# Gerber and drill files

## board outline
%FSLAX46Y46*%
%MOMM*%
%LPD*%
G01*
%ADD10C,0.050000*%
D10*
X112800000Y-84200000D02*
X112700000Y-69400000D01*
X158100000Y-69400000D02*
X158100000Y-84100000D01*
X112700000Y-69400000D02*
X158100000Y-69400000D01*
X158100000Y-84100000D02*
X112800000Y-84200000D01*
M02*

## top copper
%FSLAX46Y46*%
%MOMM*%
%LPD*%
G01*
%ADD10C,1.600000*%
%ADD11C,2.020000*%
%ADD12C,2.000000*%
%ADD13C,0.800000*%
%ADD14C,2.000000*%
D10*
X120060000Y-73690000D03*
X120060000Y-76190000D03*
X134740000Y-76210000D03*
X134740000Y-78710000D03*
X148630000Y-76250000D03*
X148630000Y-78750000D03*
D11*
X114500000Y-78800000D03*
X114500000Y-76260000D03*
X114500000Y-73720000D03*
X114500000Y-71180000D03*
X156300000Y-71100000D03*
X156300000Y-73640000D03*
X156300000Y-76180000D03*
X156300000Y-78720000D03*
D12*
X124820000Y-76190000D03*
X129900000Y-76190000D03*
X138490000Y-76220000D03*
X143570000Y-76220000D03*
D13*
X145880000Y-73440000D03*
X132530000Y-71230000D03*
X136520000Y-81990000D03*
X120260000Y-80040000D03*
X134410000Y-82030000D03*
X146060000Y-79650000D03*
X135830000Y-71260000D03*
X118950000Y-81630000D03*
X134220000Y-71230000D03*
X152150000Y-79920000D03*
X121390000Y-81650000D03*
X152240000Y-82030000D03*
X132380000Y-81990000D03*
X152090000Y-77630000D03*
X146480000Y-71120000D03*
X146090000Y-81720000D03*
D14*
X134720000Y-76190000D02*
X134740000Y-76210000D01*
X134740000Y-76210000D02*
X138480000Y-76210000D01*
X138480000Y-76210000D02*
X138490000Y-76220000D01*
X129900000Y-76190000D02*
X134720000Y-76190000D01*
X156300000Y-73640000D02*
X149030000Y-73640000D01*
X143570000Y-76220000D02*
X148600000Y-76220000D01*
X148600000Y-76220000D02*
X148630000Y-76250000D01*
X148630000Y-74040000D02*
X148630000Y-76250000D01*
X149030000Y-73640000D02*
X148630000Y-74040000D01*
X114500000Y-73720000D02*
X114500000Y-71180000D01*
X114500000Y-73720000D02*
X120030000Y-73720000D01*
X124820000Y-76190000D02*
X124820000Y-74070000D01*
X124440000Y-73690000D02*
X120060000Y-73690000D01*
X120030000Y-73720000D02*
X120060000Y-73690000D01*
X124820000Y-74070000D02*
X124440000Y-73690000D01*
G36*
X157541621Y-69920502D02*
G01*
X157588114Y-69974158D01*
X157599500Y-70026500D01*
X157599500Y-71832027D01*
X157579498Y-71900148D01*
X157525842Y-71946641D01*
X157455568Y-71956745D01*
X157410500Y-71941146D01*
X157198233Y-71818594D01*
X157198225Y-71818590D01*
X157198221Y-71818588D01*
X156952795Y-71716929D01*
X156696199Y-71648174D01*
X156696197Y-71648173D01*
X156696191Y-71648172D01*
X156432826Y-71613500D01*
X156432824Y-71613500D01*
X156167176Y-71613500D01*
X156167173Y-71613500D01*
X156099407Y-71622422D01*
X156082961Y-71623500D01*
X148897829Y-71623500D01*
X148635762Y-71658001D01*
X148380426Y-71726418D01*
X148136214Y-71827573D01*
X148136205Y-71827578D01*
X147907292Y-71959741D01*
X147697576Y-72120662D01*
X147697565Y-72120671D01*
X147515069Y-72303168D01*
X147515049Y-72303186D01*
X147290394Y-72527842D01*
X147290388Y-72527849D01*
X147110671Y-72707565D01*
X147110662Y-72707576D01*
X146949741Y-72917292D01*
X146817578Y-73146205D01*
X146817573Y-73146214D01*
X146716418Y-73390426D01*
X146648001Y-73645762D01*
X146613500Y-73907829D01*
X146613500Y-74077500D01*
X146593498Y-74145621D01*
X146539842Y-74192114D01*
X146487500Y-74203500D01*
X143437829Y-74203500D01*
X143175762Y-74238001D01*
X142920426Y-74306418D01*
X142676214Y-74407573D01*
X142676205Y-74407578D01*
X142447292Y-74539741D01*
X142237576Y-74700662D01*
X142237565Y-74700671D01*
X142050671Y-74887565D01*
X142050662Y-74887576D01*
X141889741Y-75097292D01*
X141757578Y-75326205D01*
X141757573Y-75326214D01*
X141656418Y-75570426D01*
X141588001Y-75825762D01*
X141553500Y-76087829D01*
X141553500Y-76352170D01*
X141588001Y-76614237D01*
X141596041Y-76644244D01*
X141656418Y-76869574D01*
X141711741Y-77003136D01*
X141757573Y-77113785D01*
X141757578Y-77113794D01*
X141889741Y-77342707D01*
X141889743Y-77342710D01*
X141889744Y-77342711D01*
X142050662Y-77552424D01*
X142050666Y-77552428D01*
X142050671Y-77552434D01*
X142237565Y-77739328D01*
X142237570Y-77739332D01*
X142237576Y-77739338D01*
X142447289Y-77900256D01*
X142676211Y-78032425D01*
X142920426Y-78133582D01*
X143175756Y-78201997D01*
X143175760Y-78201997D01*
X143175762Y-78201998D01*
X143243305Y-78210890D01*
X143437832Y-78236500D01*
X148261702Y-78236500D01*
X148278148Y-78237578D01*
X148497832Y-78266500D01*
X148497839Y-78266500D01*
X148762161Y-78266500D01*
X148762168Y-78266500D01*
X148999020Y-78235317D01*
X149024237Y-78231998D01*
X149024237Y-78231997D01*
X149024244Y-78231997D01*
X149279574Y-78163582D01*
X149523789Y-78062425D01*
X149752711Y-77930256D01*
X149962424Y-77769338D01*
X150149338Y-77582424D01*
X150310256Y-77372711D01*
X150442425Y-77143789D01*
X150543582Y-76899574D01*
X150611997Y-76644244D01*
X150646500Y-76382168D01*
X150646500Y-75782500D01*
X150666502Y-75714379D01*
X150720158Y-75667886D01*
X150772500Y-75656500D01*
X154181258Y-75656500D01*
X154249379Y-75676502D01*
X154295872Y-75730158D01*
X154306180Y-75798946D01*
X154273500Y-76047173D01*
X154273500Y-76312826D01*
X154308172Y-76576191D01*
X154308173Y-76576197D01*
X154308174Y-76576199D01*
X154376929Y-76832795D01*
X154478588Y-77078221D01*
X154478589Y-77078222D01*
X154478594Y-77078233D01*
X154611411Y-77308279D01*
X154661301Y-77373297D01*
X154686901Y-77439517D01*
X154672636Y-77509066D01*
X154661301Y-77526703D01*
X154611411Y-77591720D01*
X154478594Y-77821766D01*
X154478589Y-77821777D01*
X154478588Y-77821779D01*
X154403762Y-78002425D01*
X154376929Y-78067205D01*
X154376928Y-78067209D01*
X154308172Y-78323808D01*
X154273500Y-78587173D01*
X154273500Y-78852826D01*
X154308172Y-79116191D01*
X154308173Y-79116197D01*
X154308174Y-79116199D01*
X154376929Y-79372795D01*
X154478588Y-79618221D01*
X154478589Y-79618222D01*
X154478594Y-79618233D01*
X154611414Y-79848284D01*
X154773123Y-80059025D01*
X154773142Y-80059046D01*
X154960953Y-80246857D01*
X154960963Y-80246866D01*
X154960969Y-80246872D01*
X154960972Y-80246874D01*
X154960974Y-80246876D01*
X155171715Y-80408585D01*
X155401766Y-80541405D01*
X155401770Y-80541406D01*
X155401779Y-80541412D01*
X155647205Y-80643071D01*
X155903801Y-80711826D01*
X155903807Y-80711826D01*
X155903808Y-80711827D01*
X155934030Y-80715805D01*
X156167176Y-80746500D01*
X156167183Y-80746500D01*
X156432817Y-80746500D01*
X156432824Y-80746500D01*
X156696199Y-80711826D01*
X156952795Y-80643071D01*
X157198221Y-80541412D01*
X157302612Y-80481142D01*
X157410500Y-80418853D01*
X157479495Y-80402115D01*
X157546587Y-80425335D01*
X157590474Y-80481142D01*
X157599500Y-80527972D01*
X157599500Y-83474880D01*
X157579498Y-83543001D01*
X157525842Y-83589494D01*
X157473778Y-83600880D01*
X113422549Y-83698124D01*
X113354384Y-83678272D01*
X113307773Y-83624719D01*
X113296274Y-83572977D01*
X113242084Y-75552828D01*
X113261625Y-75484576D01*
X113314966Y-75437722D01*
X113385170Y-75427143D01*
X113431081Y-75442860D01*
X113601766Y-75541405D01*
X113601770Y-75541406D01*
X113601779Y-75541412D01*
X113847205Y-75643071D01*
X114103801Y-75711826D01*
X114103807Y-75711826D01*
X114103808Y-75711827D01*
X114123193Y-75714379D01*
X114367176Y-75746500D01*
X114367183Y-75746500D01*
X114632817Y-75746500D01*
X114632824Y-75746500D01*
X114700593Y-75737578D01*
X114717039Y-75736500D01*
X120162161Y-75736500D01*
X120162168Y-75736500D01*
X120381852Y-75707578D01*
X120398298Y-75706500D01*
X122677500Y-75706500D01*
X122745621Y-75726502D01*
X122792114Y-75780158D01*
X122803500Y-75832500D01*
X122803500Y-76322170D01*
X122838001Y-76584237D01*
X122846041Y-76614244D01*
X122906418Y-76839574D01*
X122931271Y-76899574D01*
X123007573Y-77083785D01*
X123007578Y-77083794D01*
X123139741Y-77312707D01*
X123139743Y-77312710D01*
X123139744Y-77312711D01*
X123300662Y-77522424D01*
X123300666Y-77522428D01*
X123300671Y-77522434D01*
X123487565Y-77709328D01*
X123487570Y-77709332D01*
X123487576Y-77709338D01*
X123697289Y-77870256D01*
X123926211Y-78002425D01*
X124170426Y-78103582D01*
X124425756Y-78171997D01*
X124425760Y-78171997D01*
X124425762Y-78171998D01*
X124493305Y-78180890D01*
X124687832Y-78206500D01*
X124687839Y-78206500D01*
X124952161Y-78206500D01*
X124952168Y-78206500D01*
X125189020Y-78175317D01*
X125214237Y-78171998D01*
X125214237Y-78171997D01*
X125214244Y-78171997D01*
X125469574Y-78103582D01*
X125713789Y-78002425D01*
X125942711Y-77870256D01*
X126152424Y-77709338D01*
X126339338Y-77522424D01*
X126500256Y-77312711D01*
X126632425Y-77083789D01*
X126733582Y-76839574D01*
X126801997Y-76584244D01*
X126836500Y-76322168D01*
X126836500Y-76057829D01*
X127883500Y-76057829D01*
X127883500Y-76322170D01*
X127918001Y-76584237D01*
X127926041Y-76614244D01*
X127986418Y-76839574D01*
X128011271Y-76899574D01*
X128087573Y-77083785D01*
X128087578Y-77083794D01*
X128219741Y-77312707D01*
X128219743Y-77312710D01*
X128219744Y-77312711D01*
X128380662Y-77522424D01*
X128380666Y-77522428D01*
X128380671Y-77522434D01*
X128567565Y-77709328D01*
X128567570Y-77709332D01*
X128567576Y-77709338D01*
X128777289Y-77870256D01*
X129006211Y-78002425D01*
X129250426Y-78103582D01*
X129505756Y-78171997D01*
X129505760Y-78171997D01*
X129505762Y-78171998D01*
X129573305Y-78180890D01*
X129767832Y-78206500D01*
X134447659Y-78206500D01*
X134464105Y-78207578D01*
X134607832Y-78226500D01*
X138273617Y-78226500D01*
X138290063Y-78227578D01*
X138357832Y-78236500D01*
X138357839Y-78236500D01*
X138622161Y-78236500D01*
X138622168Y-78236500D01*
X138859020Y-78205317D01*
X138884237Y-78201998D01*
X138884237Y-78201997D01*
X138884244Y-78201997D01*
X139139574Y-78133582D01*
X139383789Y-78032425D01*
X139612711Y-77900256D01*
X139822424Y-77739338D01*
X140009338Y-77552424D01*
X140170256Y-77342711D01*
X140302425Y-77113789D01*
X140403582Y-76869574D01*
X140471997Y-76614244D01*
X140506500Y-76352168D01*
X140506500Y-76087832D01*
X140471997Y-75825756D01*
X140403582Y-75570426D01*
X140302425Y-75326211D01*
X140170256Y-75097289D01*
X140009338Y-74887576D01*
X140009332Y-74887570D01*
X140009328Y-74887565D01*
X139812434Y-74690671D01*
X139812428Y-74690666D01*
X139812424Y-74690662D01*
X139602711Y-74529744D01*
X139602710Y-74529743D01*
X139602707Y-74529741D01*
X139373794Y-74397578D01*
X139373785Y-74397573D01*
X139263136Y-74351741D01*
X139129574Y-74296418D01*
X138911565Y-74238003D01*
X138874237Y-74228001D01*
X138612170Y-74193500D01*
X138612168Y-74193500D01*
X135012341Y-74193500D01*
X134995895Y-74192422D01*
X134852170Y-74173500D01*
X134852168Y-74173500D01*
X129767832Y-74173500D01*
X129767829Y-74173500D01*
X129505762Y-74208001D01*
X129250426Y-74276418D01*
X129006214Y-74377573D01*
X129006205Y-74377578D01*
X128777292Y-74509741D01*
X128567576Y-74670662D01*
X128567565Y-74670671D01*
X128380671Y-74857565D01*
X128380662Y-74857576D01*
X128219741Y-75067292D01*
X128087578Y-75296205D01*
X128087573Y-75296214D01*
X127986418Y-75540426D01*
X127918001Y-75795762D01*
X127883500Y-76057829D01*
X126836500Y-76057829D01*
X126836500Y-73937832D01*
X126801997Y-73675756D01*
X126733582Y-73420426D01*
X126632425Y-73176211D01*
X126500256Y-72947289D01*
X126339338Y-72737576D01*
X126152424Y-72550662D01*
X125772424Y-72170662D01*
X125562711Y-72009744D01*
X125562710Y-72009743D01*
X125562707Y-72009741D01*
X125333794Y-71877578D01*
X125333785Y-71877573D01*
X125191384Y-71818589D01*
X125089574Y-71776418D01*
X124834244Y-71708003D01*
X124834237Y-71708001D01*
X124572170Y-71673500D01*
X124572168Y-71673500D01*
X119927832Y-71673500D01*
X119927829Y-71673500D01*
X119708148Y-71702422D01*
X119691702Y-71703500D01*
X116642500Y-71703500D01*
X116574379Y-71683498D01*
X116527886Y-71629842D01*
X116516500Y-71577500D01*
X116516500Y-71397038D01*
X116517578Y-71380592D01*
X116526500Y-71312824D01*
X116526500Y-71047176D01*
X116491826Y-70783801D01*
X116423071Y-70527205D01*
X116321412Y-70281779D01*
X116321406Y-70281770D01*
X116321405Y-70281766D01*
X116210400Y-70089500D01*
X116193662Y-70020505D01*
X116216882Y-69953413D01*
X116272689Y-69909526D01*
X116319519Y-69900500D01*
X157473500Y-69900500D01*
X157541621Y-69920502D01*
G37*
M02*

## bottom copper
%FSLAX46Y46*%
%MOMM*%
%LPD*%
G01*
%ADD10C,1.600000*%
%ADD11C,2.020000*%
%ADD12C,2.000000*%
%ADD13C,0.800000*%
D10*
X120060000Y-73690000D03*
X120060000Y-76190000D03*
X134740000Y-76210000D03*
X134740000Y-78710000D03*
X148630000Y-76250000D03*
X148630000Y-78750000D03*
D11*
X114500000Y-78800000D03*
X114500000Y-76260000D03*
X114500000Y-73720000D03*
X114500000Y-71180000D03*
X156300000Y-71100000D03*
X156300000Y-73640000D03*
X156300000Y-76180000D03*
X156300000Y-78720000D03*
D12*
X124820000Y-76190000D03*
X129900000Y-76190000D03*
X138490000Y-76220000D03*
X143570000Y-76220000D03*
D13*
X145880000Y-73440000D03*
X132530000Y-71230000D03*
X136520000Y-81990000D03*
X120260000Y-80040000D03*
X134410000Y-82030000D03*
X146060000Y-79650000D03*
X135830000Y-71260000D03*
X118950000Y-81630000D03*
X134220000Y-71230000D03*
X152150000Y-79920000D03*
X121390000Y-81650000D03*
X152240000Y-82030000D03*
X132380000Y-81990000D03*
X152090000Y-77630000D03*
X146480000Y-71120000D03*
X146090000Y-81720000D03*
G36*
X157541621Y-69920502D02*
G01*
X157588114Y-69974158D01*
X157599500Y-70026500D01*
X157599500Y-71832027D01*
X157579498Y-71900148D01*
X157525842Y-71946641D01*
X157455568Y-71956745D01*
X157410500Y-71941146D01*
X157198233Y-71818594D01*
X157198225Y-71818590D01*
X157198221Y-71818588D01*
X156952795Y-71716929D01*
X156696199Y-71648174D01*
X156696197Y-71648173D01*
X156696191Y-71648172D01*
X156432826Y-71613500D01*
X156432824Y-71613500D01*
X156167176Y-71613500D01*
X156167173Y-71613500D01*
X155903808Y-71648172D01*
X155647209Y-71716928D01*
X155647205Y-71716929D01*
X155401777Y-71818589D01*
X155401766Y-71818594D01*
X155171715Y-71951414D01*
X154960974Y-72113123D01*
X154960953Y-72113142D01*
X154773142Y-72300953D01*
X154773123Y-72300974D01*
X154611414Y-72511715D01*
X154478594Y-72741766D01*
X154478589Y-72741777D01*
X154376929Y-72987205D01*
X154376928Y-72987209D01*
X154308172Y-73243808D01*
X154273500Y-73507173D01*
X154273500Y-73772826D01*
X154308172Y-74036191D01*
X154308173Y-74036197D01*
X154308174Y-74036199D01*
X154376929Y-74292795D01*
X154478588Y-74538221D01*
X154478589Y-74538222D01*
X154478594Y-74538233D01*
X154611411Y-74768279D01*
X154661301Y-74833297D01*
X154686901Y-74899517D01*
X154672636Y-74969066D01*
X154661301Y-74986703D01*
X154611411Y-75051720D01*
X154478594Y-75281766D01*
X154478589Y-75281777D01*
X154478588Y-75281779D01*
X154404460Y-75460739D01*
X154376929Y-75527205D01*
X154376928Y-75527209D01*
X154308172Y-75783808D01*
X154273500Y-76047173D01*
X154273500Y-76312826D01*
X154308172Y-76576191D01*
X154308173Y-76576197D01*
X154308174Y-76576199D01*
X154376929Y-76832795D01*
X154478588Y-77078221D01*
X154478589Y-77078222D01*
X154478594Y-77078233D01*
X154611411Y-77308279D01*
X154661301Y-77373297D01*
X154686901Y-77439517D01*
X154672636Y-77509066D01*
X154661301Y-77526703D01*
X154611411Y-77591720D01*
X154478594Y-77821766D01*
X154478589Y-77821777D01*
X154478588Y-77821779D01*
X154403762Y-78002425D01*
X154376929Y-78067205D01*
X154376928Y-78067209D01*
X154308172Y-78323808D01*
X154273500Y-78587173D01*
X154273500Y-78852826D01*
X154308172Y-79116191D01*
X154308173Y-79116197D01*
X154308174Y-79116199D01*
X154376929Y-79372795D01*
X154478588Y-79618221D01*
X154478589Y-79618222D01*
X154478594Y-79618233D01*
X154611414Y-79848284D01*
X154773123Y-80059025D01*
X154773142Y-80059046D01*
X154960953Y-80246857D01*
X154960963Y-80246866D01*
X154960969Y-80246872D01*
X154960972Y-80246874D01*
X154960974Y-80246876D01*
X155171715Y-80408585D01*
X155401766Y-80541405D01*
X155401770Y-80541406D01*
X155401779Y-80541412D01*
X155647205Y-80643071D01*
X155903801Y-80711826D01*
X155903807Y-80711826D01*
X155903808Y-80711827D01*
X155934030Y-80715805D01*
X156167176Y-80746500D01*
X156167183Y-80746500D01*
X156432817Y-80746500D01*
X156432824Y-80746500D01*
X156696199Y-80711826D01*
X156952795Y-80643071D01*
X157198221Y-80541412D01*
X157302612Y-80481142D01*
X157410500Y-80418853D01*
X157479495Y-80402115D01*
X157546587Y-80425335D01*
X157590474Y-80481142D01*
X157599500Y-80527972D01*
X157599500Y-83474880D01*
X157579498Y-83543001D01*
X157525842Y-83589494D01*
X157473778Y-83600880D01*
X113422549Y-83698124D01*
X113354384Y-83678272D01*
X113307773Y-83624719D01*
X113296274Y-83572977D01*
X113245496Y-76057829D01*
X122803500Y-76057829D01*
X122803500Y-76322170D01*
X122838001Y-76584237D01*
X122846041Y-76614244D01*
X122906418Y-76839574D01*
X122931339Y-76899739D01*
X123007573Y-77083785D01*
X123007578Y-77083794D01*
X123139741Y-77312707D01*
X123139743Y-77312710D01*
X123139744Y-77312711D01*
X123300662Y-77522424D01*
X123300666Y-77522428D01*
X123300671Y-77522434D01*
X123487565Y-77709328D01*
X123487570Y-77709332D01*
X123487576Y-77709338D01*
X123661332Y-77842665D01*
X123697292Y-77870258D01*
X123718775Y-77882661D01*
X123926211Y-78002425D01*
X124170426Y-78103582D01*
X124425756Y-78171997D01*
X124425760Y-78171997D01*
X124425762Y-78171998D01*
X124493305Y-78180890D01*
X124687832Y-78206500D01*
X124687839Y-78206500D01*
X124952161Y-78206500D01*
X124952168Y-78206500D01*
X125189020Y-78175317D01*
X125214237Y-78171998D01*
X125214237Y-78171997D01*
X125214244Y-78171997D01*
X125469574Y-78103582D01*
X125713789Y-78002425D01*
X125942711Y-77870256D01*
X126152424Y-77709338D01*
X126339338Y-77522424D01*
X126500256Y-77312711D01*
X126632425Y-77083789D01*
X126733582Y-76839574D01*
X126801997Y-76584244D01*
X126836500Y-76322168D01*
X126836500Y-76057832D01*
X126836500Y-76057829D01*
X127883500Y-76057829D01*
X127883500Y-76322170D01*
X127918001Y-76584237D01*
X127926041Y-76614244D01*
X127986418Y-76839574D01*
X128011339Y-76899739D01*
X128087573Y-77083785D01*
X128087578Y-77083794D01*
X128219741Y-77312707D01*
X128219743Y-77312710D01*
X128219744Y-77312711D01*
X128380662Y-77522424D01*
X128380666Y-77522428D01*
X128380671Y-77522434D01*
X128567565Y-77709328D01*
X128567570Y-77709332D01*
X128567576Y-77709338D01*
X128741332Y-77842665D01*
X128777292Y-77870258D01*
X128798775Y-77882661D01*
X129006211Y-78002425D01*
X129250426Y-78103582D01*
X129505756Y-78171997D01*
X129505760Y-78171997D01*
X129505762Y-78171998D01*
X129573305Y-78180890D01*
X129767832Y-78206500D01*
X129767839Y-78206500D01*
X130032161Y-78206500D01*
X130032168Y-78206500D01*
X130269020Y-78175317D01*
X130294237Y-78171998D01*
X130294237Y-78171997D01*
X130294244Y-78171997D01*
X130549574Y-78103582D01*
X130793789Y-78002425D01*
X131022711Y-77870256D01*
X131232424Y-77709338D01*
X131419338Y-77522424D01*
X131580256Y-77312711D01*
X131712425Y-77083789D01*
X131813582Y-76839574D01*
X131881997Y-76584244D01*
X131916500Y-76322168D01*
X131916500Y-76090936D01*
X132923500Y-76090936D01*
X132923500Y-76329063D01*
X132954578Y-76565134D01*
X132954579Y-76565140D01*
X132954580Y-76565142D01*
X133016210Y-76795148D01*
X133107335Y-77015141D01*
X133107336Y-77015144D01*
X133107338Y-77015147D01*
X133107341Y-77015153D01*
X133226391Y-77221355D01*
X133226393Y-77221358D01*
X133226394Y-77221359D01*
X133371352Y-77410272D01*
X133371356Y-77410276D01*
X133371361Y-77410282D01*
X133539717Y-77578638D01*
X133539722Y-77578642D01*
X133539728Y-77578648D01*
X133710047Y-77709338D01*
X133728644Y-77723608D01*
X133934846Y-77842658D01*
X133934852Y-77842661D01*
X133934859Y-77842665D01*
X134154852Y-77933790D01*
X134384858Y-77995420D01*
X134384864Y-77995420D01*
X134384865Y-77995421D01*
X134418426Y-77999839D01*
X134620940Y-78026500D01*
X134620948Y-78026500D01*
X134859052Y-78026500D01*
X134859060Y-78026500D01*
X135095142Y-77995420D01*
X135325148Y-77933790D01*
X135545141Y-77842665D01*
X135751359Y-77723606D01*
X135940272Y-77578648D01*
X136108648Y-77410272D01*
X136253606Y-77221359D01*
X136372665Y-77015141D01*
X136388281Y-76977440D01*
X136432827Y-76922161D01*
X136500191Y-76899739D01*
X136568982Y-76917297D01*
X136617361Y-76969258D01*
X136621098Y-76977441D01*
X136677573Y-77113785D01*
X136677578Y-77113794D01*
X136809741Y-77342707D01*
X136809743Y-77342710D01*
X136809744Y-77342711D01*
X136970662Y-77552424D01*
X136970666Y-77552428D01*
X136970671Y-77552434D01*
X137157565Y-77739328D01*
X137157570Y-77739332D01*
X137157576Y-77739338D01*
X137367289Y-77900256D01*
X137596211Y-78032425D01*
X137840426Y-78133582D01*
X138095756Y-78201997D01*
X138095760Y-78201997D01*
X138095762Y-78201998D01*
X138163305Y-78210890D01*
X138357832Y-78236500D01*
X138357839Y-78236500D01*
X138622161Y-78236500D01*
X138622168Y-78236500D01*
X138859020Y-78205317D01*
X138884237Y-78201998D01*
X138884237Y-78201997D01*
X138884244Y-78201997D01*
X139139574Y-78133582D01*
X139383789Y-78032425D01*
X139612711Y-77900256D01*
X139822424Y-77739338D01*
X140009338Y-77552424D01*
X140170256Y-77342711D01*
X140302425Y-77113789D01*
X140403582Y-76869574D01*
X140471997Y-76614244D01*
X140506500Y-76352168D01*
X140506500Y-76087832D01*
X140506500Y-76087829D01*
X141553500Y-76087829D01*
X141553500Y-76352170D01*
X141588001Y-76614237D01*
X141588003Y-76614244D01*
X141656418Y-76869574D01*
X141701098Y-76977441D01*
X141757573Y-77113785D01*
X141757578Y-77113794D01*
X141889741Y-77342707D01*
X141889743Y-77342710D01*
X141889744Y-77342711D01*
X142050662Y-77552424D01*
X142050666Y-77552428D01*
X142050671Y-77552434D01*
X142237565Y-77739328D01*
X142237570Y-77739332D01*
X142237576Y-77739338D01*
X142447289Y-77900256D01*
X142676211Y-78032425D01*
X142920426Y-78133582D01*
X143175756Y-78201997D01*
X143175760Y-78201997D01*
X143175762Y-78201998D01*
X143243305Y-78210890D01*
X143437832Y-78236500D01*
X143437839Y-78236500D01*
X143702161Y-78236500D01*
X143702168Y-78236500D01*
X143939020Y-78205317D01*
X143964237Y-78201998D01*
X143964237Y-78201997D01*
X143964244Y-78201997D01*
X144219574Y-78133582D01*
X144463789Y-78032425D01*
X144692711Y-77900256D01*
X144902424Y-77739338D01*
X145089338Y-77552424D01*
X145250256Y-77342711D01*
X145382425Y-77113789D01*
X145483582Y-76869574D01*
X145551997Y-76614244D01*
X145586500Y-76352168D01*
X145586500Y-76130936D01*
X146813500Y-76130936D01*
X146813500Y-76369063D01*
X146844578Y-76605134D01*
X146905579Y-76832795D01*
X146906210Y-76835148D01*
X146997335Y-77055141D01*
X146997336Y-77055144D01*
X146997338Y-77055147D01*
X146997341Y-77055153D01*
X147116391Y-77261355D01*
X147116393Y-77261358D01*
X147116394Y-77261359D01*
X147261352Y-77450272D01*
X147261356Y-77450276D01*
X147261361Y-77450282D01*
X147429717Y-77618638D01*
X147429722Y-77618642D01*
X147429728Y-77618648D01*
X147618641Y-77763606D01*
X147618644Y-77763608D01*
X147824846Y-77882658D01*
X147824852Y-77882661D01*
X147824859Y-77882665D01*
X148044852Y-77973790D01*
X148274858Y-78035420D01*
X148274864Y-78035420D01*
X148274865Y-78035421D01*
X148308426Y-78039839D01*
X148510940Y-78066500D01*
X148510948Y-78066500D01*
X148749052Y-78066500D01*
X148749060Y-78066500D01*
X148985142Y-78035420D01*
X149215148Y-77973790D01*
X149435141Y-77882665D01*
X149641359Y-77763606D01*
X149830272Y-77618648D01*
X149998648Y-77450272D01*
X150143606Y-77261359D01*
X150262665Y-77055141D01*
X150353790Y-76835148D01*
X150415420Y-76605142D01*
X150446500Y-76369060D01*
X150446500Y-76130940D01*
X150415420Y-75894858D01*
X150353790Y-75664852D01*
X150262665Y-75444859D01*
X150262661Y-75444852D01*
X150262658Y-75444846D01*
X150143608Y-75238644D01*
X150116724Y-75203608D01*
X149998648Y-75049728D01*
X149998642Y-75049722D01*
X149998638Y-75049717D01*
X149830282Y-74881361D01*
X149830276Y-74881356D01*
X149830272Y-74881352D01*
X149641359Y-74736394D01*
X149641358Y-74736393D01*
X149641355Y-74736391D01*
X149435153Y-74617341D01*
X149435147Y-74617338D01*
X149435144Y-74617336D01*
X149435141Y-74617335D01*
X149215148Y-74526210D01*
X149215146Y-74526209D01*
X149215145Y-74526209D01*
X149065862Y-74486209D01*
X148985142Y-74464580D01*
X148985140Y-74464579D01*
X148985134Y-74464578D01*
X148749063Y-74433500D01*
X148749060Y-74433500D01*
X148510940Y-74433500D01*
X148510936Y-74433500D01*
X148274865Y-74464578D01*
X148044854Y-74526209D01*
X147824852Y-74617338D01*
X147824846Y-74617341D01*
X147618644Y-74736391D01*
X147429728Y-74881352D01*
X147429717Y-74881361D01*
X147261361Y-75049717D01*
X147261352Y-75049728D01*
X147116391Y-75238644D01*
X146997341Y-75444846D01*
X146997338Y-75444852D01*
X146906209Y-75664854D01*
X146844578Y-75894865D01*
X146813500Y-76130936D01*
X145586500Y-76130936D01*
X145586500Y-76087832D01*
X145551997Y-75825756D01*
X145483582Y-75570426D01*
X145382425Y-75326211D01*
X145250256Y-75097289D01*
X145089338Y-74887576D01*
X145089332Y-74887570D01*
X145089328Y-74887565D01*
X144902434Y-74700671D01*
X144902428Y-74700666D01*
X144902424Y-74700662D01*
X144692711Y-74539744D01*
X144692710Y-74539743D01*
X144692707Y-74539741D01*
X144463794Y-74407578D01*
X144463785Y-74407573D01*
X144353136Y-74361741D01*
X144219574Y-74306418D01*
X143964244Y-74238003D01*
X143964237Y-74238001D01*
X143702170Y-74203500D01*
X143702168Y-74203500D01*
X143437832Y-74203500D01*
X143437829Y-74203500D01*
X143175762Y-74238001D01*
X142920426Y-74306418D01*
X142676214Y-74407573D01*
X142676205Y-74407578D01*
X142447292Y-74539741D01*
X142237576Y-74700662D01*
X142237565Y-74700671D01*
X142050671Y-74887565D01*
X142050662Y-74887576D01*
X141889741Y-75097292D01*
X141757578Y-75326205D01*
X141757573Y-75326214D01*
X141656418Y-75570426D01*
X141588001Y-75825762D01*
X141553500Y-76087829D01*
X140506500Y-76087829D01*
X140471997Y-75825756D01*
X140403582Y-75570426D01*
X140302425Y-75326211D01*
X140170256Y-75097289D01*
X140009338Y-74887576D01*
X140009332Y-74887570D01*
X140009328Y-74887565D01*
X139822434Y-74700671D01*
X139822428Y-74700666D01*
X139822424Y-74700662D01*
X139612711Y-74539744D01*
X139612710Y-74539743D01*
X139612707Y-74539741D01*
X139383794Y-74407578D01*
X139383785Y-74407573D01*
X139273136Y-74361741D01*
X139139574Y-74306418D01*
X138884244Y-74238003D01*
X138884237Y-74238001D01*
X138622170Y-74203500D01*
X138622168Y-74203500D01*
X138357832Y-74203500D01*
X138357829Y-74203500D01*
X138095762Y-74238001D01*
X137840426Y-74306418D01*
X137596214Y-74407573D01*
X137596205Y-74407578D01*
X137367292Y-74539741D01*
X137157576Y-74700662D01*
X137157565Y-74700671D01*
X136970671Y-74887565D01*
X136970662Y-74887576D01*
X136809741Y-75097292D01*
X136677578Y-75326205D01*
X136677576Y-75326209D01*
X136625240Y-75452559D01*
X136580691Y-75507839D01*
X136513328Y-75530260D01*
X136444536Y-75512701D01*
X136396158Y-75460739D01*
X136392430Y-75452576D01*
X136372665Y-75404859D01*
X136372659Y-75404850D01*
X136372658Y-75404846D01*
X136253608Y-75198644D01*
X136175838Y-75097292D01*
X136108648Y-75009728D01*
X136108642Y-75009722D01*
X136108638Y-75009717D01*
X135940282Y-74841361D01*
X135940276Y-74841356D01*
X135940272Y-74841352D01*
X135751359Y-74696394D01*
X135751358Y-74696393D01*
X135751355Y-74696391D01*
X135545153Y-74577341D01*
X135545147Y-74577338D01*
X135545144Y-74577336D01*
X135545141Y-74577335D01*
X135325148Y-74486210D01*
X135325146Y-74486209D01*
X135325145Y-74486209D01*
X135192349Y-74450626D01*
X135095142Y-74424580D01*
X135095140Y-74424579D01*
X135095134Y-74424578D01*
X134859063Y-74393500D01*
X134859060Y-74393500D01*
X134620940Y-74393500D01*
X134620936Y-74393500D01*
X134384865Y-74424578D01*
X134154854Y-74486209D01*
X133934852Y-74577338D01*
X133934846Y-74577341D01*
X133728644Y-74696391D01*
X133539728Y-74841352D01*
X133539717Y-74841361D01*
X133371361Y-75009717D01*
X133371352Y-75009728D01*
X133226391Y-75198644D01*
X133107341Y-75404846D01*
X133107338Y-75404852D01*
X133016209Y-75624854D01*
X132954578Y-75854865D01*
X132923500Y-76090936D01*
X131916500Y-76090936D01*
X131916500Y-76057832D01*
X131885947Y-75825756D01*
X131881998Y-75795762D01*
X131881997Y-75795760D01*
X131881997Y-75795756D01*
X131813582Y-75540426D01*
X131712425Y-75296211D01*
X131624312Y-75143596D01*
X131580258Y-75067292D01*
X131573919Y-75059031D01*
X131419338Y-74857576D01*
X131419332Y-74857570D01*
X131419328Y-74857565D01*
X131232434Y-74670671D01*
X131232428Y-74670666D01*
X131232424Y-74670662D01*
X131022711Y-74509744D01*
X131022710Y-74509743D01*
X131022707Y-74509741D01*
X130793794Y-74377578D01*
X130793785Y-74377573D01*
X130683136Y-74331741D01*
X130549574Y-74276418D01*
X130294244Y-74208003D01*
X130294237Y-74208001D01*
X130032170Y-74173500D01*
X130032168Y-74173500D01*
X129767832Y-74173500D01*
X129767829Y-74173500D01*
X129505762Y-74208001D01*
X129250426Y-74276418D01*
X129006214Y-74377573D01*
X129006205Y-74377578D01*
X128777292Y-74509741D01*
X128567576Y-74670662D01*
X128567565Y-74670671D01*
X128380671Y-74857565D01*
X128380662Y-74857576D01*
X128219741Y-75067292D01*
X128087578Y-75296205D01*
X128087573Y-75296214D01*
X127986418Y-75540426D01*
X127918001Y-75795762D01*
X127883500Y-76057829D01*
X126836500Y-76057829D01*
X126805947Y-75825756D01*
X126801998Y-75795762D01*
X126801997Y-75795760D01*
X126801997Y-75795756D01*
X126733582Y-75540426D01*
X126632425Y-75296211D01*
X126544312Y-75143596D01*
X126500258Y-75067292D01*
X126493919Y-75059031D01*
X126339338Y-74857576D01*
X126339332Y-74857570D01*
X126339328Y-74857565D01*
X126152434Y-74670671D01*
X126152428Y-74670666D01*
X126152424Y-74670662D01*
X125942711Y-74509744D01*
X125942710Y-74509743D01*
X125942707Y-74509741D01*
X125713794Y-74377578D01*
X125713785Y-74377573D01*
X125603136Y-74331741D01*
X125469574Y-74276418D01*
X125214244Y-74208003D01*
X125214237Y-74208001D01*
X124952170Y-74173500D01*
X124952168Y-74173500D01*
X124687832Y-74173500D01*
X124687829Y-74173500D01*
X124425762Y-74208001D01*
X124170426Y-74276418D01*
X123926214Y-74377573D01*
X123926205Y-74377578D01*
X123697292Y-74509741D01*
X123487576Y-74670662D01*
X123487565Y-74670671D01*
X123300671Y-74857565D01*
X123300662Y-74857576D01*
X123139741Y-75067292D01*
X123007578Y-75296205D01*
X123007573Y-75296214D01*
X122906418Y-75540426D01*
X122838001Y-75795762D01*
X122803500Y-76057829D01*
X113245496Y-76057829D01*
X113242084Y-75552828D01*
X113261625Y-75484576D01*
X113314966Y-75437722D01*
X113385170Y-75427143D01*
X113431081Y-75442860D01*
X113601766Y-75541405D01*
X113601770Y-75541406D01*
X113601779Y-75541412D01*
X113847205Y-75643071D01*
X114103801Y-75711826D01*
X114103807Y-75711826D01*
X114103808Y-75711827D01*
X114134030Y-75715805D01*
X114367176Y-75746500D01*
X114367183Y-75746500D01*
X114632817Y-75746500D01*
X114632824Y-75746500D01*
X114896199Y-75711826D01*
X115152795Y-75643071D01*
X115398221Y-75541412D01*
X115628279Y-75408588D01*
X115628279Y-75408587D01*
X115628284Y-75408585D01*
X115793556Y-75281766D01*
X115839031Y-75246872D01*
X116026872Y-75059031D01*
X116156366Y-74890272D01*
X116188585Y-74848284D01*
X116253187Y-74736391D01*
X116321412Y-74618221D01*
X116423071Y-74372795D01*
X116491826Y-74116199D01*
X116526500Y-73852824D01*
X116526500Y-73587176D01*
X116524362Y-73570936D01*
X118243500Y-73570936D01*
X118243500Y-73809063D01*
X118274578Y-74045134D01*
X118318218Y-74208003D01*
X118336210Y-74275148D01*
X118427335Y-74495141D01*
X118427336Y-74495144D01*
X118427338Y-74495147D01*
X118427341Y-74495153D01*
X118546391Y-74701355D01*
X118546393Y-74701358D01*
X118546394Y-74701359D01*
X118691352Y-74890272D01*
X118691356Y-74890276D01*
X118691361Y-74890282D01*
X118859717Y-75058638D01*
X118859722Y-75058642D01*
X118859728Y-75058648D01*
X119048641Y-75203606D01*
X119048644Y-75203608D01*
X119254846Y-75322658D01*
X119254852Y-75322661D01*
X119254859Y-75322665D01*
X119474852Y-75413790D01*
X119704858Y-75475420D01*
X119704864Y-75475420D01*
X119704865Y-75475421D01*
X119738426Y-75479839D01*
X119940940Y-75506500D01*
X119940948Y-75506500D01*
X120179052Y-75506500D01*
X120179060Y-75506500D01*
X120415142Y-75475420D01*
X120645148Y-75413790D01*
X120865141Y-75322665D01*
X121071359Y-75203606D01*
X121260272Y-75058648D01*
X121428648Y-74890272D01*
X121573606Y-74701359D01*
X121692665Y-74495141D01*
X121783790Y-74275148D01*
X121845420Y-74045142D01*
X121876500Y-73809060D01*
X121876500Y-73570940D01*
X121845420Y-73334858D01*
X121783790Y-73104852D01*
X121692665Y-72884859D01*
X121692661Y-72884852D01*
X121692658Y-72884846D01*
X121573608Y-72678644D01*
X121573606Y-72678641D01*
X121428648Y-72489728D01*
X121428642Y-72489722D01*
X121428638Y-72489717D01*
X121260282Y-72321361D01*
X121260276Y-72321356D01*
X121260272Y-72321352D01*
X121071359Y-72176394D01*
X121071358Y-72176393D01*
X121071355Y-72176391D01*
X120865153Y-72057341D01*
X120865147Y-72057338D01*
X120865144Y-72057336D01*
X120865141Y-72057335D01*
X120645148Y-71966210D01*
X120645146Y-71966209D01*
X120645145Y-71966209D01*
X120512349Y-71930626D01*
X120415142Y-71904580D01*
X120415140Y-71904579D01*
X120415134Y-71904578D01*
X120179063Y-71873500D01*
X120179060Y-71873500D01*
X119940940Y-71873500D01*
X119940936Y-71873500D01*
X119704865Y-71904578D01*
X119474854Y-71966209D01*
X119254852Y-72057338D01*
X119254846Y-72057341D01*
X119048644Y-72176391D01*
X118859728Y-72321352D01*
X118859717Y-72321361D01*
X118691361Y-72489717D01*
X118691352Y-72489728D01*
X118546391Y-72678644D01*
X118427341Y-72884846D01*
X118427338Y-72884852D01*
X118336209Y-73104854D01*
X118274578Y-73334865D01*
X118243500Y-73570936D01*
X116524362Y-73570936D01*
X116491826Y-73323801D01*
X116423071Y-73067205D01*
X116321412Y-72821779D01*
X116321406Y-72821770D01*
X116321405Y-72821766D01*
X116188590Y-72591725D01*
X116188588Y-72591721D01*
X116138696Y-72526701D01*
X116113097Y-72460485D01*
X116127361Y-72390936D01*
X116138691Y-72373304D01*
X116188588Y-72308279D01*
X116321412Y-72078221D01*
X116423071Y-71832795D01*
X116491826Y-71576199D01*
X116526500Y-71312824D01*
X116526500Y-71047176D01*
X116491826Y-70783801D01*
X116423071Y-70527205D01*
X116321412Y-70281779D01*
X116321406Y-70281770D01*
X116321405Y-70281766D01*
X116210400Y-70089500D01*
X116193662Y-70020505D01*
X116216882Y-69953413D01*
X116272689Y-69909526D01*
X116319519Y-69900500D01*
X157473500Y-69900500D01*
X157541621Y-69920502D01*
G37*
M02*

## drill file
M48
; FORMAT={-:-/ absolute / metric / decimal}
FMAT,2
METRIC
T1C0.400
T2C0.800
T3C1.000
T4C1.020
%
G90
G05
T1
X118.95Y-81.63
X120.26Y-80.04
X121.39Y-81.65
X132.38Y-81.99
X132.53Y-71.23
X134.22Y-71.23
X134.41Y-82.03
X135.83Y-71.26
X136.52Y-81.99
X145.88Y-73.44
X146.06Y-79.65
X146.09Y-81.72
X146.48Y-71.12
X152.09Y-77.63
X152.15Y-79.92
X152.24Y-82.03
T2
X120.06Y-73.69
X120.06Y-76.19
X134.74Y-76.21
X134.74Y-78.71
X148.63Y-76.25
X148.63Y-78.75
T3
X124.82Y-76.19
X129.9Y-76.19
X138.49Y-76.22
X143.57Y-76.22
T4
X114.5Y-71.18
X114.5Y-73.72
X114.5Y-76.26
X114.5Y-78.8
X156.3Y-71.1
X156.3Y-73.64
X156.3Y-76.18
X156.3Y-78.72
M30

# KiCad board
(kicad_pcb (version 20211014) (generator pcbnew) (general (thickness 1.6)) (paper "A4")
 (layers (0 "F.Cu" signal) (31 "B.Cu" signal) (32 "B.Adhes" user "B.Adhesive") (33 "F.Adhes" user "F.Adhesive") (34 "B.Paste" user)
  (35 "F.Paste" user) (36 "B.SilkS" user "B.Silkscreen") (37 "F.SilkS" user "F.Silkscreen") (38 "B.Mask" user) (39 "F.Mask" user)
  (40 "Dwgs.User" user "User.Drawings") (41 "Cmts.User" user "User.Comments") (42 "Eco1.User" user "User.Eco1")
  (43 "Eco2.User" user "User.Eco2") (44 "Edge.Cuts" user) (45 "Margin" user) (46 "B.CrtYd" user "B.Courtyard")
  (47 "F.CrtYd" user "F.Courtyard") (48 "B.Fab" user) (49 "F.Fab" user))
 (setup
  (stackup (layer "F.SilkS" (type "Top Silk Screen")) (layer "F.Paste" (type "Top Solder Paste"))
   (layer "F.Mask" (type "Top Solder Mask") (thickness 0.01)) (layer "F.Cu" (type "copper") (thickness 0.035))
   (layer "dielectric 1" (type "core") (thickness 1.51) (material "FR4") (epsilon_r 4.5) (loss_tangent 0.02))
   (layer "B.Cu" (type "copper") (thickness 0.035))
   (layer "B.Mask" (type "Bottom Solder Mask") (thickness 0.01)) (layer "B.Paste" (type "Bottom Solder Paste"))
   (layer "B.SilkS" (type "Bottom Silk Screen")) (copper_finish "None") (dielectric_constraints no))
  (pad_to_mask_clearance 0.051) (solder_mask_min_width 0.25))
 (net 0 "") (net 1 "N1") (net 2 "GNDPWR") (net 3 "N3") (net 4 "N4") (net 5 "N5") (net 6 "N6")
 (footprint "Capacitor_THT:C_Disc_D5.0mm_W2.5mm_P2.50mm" (layer "F.Cu") (at 120.06 73.69 -90)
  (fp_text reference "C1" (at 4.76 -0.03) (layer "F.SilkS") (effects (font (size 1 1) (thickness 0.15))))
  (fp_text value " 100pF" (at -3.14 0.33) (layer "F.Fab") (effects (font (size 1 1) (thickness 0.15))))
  (pad "1" thru_hole circle locked (at 0 0 270) (size 1.6 1.6) (drill 0.8) (layers *.Cu *.Mask) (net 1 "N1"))
  (pad "2" thru_hole circle locked (at 2.5 0 270) (size 1.6 1.6) (drill 0.8) (layers *.Cu *.Mask) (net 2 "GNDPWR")))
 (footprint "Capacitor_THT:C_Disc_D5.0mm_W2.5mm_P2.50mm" (layer "F.Cu") (at 134.74 76.21 -90)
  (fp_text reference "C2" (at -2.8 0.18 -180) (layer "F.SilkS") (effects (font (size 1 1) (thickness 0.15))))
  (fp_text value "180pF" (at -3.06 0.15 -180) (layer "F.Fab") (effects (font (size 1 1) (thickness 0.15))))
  (pad "1" thru_hole circle locked (at 0 0 270) (size 1.6 1.6) (drill 0.8) (layers *.Cu *.Mask) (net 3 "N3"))
  (pad "2" thru_hole circle locked (at 2.5 0 270) (size 1.6 1.6) (drill 0.8) (layers *.Cu *.Mask) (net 2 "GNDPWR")))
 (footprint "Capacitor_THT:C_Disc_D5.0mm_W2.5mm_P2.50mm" (layer "F.Cu") (at 148.63 76.25 -90)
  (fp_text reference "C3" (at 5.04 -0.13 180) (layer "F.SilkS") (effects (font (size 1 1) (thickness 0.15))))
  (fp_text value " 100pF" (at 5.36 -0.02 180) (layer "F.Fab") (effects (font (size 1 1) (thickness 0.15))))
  (pad "1" thru_hole circle locked (at 0 0 270) (size 1.6 1.6) (drill 0.8) (layers *.Cu *.Mask) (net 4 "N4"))
  (pad "2" thru_hole circle locked (at 2.5 0 270) (size 1.6 1.6) (drill 0.8) (layers *.Cu *.Mask) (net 2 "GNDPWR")))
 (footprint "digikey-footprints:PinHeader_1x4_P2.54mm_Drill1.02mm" (layer "F.Cu") (at 114.5 78.8 90)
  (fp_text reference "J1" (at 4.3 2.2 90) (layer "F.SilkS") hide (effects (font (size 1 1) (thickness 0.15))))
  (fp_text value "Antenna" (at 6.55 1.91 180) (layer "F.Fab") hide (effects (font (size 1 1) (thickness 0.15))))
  (pad "1" thru_hole circle locked (at 0 0 90) (size 2.02 2.02) (drill 1.02) (layers *.Cu *.Mask) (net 2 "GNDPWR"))
  (pad "2" thru_hole circle locked (at 2.54 0 90) (size 2.02 2.02) (drill 1.02) (layers *.Cu *.Mask) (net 2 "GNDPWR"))
  (pad "3" thru_hole circle locked (at 5.08 0 90) (size 2.02 2.02) (drill 1.02) (layers *.Cu *.Mask) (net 1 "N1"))
  (pad "4" thru_hole circle locked (at 7.62 0 90) (size 2.02 2.02) (drill 1.02) (layers *.Cu *.Mask) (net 1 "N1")))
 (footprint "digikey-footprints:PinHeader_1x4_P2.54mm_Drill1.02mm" (layer "F.Cu") (at 156.3 71.1 -90)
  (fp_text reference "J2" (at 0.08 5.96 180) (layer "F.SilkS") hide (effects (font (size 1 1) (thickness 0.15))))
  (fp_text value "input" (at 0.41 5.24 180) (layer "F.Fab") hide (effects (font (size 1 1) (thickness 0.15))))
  (pad "1" thru_hole circle locked (at 0 0 270) (size 2.02 2.02) (drill 1.02) (layers *.Cu *.Mask) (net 2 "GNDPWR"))
  (pad "2" thru_hole circle locked (at 2.54 0 270) (size 2.02 2.02) (drill 1.02) (layers *.Cu *.Mask) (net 4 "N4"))
  (pad "3" thru_hole circle locked (at 5.08 0 270) (size 2.02 2.02) (drill 1.02) (layers *.Cu *.Mask) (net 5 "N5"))
  (pad "4" thru_hole circle locked (at 7.62 0 270) (size 2.02 2.02) (drill 1.02) (layers *.Cu *.Mask) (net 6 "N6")))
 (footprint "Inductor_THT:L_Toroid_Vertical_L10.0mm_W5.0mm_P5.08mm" (layer "F.Cu") (at 124.82 76.19 90)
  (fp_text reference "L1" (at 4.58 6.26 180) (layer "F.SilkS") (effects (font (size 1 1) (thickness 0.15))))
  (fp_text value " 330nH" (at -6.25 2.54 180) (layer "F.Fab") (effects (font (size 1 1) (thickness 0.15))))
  (pad "1" thru_hole circle locked (at 0 0 90) (size 2 2) (drill 1) (layers *.Cu *.Mask) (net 1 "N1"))
  (pad "2" thru_hole circle locked (at 0 5.08 90) (size 2 2) (drill 1) (layers *.Cu *.Mask) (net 3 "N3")))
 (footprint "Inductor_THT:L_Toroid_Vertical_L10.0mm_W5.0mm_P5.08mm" (layer "F.Cu") (at 138.49 76.22 90)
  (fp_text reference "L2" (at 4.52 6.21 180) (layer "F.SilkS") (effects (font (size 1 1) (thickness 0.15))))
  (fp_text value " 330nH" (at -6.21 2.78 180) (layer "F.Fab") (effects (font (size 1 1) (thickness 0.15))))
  (pad "1" thru_hole circle locked (at 0 0 90) (size 2 2) (drill 1) (layers *.Cu *.Mask) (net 3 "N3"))
  (pad "2" thru_hole circle locked (at 0 5.08 90) (size 2 2) (drill 1) (layers *.Cu *.Mask) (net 4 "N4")))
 (gr_line (start 112.8 84.2) (end 112.7 69.4) (layer "Edge.Cuts") (width 0.05))
 (gr_line (start 158.1 69.4) (end 158.1 84.1) (layer "Edge.Cuts") (width 0.05))
 (gr_line (start 112.7 69.4) (end 158.1 69.4) (layer "Edge.Cuts") (width 0.05))
 (gr_line (start 158.1 84.1) (end 112.8 84.2) (layer "Edge.Cuts") (width 0.05))
 (via (at 145.88 73.44) (size 0.8) (drill 0.4) (layers "F.Cu" "B.Cu") (free) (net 2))
 (via (at 132.53 71.23) (size 0.8) (drill 0.4) (layers "F.Cu" "B.Cu") (free) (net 2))
 (via (at 136.52 81.99) (size 0.8) (drill 0.4) (layers "F.Cu" "B.Cu") (free) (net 2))
 (via (at 120.26 80.04) (size 0.8) (drill 0.4) (layers "F.Cu" "B.Cu") (free) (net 2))
 (via (at 134.41 82.03) (size 0.8) (drill 0.4) (layers "F.Cu" "B.Cu") (free) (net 2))
 (via (at 146.06 79.65) (size 0.8) (drill 0.4) (layers "F.Cu" "B.Cu") (free) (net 2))
 (via (at 135.83 71.26) (size 0.8) (drill 0.4) (layers "F.Cu" "B.Cu") (free) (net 2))
 (via (at 118.95 81.63) (size 0.8) (drill 0.4) (layers "F.Cu" "B.Cu") (free) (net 2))
 (via (at 134.22 71.23) (size 0.8) (drill 0.4) (layers "F.Cu" "B.Cu") (free) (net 2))
 (via (at 152.15 79.92) (size 0.8) (drill 0.4) (layers "F.Cu" "B.Cu") (free) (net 2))
 (via (at 121.39 81.65) (size 0.8) (drill 0.4) (layers "F.Cu" "B.Cu") (free) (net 2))
 (via (at 152.24 82.03) (size 0.8) (drill 0.4) (layers "F.Cu" "B.Cu") (free) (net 2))
 (via (at 132.38 81.99) (size 0.8) (drill 0.4) (layers "F.Cu" "B.Cu") (free) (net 2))
 (via (at 152.09 77.63) (size 0.8) (drill 0.4) (layers "F.Cu" "B.Cu") (free) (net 2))
 (via (at 146.48 71.12) (size 0.8) (drill 0.4) (layers "F.Cu" "B.Cu") (free) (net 2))
 (via (at 146.09 81.72) (size 0.8) (drill 0.4) (layers "F.Cu" "B.Cu") (free) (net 2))
 (segment (start 134.72 76.19) (end 134.74 76.21) (width 2) (layer "F.Cu") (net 3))
 (segment (start 134.74 76.21) (end 138.48 76.21) (width 2) (layer "F.Cu") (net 3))
 (segment (start 138.48 76.21) (end 138.49 76.22) (width 2) (layer "F.Cu") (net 3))
 (segment (start 129.9 76.19) (end 134.72 76.19) (width 2) (layer "F.Cu") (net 3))
 (segment (start 156.3 73.64) (end 149.03 73.64) (width 2) (layer "F.Cu") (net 4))
 (segment (start 143.57 76.22) (end 148.6 76.22) (width 2) (layer "F.Cu") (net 4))
 (segment (start 148.6 76.22) (end 148.63 76.25) (width 2) (layer "F.Cu") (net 4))
 (segment (start 148.63 74.04) (end 148.63 76.25) (width 2) (layer "F.Cu") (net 4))
 (segment (start 149.03 73.64) (end 148.63 74.04) (width 2) (layer "F.Cu") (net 4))
 (segment (start 114.5 73.72) (end 114.5 71.18) (width 2) (layer "F.Cu") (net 1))
 (segment (start 114.5 73.72) (end 120.03 73.72) (width 2) (layer "F.Cu") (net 1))
 (segment (start 124.82 76.19) (end 124.82 74.07) (width 2) (layer "F.Cu") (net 1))
 (segment (start 124.44 73.69) (end 120.06 73.69) (width 2) (layer "F.Cu") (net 1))
 (segment (start 120.03 73.72) (end 120.06 73.69) (width 2) (layer "F.Cu") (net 1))
 (segment (start 124.82 74.07) (end 124.44 73.69) (width 2) (layer "F.Cu") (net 1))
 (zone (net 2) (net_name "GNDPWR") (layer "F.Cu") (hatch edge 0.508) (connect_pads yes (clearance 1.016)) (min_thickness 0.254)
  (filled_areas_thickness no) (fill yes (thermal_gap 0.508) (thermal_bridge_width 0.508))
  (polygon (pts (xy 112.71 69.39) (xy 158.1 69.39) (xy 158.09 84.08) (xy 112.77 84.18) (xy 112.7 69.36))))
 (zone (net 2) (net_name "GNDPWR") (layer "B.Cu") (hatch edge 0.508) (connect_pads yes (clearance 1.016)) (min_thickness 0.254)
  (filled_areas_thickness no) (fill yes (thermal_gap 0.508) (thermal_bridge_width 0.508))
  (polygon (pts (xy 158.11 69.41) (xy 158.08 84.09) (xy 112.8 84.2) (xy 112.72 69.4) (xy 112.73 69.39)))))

